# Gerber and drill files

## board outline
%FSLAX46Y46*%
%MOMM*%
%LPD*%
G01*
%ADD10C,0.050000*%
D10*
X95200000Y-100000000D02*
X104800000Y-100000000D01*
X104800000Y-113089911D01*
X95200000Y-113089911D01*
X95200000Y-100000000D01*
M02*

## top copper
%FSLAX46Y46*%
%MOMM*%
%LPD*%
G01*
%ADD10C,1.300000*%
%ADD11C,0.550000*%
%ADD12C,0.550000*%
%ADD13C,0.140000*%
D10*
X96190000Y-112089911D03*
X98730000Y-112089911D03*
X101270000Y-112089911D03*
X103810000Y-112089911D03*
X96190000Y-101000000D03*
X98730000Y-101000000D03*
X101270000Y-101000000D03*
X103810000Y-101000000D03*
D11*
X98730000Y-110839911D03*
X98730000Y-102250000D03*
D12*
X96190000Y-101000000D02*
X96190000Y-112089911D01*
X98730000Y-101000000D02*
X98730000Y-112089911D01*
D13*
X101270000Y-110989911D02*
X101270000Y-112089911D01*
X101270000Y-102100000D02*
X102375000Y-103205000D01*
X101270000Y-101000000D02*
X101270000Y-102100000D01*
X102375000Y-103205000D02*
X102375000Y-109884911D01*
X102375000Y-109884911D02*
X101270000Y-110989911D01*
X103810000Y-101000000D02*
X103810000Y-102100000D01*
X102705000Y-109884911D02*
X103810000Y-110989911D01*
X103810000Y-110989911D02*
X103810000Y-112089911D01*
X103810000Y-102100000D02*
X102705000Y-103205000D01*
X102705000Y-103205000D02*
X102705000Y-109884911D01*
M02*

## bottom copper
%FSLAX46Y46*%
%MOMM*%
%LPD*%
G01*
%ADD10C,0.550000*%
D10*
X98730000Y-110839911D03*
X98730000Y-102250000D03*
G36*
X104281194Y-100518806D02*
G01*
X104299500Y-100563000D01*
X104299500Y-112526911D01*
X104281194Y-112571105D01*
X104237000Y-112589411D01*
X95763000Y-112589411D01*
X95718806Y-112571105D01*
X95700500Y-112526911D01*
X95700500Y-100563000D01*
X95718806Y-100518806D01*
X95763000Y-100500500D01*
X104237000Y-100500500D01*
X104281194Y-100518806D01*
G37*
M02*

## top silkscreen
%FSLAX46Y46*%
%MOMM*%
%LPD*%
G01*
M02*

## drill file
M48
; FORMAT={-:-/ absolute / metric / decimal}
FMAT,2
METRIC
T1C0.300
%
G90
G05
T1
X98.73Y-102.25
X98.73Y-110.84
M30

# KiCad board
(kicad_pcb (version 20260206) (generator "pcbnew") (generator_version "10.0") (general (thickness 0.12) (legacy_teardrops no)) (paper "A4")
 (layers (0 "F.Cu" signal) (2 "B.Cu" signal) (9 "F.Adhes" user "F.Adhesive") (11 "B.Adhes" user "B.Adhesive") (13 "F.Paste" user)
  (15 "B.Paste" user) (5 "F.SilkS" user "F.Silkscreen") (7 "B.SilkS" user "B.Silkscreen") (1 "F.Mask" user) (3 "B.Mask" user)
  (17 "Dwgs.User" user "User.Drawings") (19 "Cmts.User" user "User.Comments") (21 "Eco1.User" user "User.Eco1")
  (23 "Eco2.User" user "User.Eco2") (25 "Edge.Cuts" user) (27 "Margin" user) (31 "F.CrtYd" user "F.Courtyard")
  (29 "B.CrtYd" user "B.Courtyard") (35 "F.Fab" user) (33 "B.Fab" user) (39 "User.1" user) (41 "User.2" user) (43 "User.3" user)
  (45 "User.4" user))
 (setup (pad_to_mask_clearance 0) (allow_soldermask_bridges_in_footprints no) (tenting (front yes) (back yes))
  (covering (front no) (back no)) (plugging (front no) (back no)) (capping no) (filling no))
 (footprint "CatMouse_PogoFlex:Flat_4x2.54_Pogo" (layer "F.Cu") (at 100 112.089911)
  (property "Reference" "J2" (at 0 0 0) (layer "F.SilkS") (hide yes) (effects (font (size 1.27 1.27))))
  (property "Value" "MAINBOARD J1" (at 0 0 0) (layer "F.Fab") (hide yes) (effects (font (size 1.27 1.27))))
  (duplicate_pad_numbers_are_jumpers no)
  (pad "1" smd circle (at -3.81 0) (size 1.3 1.3) (layers "F.Cu" "F.Mask") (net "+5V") (solder_mask_margin 0.1))
  (pad "2" smd circle (at -1.27 0) (size 1.3 1.3) (layers "F.Cu" "F.Mask") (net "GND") (solder_mask_margin 0.1))
  (pad "3" smd circle (at 1.27 0) (size 1.3 1.3) (layers "F.Cu" "F.Mask") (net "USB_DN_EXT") (solder_mask_margin 0.1))
  (pad "4" smd circle (at 3.81 0) (size 1.3 1.3) (layers "F.Cu" "F.Mask") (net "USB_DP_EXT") (solder_mask_margin 0.1)))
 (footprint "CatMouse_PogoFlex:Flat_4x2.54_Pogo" (layer "F.Cu") (at 100 101)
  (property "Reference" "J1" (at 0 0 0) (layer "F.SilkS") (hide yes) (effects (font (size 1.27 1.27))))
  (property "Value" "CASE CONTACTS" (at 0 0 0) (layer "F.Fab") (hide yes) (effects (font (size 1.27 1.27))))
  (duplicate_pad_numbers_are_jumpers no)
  (pad "1" smd circle (at -3.81 0) (size 1.3 1.3) (layers "F.Cu" "F.Mask") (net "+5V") (solder_mask_margin 0.1))
  (pad "2" smd circle (at -1.27 0) (size 1.3 1.3) (layers "F.Cu" "F.Mask") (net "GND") (solder_mask_margin 0.1))
  (pad "3" smd circle (at 1.27 0) (size 1.3 1.3) (layers "F.Cu" "F.Mask") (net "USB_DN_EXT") (solder_mask_margin 0.1))
  (pad "4" smd circle (at 3.81 0) (size 1.3 1.3) (layers "F.Cu" "F.Mask") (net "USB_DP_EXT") (solder_mask_margin 0.1)))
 (gr_rect (start 95.2 100) (end 104.8 113.089911) (stroke (width 0.05) (type default)) (fill no) (layer "Edge.Cuts"))
 (segment (start 96.19 101) (end 96.19 112.089911) (width 0.55) (layer "F.Cu") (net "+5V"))
 (segment (start 98.73 101) (end 98.73 112.089911) (width 0.55) (layer "F.Cu") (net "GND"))
 (via (at 98.73 110.839911) (size 0.55) (drill 0.3) (layers "F.Cu" "B.Cu") (tenting (front yes) (back yes)) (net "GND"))
 (via (at 98.73 102.25) (size 0.55) (drill 0.3) (layers "F.Cu" "B.Cu") (tenting (front yes) (back yes)) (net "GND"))
 (segment (start 101.27 110.989911) (end 101.27 112.089911) (width 0.14) (layer "F.Cu") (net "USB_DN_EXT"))
 (segment (start 101.27 102.1) (end 102.375 103.205) (width 0.14) (layer "F.Cu") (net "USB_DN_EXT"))
 (segment (start 101.27 101) (end 101.27 102.1) (width 0.14) (layer "F.Cu") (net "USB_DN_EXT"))
 (segment (start 102.375 103.205) (end 102.375 109.884911) (width 0.14) (layer "F.Cu") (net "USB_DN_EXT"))
 (segment (start 102.375 109.884911) (end 101.27 110.989911) (width 0.14) (layer "F.Cu") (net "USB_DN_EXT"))
 (segment (start 103.81 101) (end 103.81 102.1) (width 0.14) (layer "F.Cu") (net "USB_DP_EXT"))
 (segment (start 102.705 109.884911) (end 103.81 110.989911) (width 0.14) (layer "F.Cu") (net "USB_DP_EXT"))
 (segment (start 103.81 110.989911) (end 103.81 112.089911) (width 0.14) (layer "F.Cu") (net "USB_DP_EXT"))
 (segment (start 103.81 102.1) (end 102.705 103.205) (width 0.14) (layer "F.Cu") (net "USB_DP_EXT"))
 (segment (start 102.705 103.205) (end 102.705 109.884911) (width 0.14) (layer "F.Cu") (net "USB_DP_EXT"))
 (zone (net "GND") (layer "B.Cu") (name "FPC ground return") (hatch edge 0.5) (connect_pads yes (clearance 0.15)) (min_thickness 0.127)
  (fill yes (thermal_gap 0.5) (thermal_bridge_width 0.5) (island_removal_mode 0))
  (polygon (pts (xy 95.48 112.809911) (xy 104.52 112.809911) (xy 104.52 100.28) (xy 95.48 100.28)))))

